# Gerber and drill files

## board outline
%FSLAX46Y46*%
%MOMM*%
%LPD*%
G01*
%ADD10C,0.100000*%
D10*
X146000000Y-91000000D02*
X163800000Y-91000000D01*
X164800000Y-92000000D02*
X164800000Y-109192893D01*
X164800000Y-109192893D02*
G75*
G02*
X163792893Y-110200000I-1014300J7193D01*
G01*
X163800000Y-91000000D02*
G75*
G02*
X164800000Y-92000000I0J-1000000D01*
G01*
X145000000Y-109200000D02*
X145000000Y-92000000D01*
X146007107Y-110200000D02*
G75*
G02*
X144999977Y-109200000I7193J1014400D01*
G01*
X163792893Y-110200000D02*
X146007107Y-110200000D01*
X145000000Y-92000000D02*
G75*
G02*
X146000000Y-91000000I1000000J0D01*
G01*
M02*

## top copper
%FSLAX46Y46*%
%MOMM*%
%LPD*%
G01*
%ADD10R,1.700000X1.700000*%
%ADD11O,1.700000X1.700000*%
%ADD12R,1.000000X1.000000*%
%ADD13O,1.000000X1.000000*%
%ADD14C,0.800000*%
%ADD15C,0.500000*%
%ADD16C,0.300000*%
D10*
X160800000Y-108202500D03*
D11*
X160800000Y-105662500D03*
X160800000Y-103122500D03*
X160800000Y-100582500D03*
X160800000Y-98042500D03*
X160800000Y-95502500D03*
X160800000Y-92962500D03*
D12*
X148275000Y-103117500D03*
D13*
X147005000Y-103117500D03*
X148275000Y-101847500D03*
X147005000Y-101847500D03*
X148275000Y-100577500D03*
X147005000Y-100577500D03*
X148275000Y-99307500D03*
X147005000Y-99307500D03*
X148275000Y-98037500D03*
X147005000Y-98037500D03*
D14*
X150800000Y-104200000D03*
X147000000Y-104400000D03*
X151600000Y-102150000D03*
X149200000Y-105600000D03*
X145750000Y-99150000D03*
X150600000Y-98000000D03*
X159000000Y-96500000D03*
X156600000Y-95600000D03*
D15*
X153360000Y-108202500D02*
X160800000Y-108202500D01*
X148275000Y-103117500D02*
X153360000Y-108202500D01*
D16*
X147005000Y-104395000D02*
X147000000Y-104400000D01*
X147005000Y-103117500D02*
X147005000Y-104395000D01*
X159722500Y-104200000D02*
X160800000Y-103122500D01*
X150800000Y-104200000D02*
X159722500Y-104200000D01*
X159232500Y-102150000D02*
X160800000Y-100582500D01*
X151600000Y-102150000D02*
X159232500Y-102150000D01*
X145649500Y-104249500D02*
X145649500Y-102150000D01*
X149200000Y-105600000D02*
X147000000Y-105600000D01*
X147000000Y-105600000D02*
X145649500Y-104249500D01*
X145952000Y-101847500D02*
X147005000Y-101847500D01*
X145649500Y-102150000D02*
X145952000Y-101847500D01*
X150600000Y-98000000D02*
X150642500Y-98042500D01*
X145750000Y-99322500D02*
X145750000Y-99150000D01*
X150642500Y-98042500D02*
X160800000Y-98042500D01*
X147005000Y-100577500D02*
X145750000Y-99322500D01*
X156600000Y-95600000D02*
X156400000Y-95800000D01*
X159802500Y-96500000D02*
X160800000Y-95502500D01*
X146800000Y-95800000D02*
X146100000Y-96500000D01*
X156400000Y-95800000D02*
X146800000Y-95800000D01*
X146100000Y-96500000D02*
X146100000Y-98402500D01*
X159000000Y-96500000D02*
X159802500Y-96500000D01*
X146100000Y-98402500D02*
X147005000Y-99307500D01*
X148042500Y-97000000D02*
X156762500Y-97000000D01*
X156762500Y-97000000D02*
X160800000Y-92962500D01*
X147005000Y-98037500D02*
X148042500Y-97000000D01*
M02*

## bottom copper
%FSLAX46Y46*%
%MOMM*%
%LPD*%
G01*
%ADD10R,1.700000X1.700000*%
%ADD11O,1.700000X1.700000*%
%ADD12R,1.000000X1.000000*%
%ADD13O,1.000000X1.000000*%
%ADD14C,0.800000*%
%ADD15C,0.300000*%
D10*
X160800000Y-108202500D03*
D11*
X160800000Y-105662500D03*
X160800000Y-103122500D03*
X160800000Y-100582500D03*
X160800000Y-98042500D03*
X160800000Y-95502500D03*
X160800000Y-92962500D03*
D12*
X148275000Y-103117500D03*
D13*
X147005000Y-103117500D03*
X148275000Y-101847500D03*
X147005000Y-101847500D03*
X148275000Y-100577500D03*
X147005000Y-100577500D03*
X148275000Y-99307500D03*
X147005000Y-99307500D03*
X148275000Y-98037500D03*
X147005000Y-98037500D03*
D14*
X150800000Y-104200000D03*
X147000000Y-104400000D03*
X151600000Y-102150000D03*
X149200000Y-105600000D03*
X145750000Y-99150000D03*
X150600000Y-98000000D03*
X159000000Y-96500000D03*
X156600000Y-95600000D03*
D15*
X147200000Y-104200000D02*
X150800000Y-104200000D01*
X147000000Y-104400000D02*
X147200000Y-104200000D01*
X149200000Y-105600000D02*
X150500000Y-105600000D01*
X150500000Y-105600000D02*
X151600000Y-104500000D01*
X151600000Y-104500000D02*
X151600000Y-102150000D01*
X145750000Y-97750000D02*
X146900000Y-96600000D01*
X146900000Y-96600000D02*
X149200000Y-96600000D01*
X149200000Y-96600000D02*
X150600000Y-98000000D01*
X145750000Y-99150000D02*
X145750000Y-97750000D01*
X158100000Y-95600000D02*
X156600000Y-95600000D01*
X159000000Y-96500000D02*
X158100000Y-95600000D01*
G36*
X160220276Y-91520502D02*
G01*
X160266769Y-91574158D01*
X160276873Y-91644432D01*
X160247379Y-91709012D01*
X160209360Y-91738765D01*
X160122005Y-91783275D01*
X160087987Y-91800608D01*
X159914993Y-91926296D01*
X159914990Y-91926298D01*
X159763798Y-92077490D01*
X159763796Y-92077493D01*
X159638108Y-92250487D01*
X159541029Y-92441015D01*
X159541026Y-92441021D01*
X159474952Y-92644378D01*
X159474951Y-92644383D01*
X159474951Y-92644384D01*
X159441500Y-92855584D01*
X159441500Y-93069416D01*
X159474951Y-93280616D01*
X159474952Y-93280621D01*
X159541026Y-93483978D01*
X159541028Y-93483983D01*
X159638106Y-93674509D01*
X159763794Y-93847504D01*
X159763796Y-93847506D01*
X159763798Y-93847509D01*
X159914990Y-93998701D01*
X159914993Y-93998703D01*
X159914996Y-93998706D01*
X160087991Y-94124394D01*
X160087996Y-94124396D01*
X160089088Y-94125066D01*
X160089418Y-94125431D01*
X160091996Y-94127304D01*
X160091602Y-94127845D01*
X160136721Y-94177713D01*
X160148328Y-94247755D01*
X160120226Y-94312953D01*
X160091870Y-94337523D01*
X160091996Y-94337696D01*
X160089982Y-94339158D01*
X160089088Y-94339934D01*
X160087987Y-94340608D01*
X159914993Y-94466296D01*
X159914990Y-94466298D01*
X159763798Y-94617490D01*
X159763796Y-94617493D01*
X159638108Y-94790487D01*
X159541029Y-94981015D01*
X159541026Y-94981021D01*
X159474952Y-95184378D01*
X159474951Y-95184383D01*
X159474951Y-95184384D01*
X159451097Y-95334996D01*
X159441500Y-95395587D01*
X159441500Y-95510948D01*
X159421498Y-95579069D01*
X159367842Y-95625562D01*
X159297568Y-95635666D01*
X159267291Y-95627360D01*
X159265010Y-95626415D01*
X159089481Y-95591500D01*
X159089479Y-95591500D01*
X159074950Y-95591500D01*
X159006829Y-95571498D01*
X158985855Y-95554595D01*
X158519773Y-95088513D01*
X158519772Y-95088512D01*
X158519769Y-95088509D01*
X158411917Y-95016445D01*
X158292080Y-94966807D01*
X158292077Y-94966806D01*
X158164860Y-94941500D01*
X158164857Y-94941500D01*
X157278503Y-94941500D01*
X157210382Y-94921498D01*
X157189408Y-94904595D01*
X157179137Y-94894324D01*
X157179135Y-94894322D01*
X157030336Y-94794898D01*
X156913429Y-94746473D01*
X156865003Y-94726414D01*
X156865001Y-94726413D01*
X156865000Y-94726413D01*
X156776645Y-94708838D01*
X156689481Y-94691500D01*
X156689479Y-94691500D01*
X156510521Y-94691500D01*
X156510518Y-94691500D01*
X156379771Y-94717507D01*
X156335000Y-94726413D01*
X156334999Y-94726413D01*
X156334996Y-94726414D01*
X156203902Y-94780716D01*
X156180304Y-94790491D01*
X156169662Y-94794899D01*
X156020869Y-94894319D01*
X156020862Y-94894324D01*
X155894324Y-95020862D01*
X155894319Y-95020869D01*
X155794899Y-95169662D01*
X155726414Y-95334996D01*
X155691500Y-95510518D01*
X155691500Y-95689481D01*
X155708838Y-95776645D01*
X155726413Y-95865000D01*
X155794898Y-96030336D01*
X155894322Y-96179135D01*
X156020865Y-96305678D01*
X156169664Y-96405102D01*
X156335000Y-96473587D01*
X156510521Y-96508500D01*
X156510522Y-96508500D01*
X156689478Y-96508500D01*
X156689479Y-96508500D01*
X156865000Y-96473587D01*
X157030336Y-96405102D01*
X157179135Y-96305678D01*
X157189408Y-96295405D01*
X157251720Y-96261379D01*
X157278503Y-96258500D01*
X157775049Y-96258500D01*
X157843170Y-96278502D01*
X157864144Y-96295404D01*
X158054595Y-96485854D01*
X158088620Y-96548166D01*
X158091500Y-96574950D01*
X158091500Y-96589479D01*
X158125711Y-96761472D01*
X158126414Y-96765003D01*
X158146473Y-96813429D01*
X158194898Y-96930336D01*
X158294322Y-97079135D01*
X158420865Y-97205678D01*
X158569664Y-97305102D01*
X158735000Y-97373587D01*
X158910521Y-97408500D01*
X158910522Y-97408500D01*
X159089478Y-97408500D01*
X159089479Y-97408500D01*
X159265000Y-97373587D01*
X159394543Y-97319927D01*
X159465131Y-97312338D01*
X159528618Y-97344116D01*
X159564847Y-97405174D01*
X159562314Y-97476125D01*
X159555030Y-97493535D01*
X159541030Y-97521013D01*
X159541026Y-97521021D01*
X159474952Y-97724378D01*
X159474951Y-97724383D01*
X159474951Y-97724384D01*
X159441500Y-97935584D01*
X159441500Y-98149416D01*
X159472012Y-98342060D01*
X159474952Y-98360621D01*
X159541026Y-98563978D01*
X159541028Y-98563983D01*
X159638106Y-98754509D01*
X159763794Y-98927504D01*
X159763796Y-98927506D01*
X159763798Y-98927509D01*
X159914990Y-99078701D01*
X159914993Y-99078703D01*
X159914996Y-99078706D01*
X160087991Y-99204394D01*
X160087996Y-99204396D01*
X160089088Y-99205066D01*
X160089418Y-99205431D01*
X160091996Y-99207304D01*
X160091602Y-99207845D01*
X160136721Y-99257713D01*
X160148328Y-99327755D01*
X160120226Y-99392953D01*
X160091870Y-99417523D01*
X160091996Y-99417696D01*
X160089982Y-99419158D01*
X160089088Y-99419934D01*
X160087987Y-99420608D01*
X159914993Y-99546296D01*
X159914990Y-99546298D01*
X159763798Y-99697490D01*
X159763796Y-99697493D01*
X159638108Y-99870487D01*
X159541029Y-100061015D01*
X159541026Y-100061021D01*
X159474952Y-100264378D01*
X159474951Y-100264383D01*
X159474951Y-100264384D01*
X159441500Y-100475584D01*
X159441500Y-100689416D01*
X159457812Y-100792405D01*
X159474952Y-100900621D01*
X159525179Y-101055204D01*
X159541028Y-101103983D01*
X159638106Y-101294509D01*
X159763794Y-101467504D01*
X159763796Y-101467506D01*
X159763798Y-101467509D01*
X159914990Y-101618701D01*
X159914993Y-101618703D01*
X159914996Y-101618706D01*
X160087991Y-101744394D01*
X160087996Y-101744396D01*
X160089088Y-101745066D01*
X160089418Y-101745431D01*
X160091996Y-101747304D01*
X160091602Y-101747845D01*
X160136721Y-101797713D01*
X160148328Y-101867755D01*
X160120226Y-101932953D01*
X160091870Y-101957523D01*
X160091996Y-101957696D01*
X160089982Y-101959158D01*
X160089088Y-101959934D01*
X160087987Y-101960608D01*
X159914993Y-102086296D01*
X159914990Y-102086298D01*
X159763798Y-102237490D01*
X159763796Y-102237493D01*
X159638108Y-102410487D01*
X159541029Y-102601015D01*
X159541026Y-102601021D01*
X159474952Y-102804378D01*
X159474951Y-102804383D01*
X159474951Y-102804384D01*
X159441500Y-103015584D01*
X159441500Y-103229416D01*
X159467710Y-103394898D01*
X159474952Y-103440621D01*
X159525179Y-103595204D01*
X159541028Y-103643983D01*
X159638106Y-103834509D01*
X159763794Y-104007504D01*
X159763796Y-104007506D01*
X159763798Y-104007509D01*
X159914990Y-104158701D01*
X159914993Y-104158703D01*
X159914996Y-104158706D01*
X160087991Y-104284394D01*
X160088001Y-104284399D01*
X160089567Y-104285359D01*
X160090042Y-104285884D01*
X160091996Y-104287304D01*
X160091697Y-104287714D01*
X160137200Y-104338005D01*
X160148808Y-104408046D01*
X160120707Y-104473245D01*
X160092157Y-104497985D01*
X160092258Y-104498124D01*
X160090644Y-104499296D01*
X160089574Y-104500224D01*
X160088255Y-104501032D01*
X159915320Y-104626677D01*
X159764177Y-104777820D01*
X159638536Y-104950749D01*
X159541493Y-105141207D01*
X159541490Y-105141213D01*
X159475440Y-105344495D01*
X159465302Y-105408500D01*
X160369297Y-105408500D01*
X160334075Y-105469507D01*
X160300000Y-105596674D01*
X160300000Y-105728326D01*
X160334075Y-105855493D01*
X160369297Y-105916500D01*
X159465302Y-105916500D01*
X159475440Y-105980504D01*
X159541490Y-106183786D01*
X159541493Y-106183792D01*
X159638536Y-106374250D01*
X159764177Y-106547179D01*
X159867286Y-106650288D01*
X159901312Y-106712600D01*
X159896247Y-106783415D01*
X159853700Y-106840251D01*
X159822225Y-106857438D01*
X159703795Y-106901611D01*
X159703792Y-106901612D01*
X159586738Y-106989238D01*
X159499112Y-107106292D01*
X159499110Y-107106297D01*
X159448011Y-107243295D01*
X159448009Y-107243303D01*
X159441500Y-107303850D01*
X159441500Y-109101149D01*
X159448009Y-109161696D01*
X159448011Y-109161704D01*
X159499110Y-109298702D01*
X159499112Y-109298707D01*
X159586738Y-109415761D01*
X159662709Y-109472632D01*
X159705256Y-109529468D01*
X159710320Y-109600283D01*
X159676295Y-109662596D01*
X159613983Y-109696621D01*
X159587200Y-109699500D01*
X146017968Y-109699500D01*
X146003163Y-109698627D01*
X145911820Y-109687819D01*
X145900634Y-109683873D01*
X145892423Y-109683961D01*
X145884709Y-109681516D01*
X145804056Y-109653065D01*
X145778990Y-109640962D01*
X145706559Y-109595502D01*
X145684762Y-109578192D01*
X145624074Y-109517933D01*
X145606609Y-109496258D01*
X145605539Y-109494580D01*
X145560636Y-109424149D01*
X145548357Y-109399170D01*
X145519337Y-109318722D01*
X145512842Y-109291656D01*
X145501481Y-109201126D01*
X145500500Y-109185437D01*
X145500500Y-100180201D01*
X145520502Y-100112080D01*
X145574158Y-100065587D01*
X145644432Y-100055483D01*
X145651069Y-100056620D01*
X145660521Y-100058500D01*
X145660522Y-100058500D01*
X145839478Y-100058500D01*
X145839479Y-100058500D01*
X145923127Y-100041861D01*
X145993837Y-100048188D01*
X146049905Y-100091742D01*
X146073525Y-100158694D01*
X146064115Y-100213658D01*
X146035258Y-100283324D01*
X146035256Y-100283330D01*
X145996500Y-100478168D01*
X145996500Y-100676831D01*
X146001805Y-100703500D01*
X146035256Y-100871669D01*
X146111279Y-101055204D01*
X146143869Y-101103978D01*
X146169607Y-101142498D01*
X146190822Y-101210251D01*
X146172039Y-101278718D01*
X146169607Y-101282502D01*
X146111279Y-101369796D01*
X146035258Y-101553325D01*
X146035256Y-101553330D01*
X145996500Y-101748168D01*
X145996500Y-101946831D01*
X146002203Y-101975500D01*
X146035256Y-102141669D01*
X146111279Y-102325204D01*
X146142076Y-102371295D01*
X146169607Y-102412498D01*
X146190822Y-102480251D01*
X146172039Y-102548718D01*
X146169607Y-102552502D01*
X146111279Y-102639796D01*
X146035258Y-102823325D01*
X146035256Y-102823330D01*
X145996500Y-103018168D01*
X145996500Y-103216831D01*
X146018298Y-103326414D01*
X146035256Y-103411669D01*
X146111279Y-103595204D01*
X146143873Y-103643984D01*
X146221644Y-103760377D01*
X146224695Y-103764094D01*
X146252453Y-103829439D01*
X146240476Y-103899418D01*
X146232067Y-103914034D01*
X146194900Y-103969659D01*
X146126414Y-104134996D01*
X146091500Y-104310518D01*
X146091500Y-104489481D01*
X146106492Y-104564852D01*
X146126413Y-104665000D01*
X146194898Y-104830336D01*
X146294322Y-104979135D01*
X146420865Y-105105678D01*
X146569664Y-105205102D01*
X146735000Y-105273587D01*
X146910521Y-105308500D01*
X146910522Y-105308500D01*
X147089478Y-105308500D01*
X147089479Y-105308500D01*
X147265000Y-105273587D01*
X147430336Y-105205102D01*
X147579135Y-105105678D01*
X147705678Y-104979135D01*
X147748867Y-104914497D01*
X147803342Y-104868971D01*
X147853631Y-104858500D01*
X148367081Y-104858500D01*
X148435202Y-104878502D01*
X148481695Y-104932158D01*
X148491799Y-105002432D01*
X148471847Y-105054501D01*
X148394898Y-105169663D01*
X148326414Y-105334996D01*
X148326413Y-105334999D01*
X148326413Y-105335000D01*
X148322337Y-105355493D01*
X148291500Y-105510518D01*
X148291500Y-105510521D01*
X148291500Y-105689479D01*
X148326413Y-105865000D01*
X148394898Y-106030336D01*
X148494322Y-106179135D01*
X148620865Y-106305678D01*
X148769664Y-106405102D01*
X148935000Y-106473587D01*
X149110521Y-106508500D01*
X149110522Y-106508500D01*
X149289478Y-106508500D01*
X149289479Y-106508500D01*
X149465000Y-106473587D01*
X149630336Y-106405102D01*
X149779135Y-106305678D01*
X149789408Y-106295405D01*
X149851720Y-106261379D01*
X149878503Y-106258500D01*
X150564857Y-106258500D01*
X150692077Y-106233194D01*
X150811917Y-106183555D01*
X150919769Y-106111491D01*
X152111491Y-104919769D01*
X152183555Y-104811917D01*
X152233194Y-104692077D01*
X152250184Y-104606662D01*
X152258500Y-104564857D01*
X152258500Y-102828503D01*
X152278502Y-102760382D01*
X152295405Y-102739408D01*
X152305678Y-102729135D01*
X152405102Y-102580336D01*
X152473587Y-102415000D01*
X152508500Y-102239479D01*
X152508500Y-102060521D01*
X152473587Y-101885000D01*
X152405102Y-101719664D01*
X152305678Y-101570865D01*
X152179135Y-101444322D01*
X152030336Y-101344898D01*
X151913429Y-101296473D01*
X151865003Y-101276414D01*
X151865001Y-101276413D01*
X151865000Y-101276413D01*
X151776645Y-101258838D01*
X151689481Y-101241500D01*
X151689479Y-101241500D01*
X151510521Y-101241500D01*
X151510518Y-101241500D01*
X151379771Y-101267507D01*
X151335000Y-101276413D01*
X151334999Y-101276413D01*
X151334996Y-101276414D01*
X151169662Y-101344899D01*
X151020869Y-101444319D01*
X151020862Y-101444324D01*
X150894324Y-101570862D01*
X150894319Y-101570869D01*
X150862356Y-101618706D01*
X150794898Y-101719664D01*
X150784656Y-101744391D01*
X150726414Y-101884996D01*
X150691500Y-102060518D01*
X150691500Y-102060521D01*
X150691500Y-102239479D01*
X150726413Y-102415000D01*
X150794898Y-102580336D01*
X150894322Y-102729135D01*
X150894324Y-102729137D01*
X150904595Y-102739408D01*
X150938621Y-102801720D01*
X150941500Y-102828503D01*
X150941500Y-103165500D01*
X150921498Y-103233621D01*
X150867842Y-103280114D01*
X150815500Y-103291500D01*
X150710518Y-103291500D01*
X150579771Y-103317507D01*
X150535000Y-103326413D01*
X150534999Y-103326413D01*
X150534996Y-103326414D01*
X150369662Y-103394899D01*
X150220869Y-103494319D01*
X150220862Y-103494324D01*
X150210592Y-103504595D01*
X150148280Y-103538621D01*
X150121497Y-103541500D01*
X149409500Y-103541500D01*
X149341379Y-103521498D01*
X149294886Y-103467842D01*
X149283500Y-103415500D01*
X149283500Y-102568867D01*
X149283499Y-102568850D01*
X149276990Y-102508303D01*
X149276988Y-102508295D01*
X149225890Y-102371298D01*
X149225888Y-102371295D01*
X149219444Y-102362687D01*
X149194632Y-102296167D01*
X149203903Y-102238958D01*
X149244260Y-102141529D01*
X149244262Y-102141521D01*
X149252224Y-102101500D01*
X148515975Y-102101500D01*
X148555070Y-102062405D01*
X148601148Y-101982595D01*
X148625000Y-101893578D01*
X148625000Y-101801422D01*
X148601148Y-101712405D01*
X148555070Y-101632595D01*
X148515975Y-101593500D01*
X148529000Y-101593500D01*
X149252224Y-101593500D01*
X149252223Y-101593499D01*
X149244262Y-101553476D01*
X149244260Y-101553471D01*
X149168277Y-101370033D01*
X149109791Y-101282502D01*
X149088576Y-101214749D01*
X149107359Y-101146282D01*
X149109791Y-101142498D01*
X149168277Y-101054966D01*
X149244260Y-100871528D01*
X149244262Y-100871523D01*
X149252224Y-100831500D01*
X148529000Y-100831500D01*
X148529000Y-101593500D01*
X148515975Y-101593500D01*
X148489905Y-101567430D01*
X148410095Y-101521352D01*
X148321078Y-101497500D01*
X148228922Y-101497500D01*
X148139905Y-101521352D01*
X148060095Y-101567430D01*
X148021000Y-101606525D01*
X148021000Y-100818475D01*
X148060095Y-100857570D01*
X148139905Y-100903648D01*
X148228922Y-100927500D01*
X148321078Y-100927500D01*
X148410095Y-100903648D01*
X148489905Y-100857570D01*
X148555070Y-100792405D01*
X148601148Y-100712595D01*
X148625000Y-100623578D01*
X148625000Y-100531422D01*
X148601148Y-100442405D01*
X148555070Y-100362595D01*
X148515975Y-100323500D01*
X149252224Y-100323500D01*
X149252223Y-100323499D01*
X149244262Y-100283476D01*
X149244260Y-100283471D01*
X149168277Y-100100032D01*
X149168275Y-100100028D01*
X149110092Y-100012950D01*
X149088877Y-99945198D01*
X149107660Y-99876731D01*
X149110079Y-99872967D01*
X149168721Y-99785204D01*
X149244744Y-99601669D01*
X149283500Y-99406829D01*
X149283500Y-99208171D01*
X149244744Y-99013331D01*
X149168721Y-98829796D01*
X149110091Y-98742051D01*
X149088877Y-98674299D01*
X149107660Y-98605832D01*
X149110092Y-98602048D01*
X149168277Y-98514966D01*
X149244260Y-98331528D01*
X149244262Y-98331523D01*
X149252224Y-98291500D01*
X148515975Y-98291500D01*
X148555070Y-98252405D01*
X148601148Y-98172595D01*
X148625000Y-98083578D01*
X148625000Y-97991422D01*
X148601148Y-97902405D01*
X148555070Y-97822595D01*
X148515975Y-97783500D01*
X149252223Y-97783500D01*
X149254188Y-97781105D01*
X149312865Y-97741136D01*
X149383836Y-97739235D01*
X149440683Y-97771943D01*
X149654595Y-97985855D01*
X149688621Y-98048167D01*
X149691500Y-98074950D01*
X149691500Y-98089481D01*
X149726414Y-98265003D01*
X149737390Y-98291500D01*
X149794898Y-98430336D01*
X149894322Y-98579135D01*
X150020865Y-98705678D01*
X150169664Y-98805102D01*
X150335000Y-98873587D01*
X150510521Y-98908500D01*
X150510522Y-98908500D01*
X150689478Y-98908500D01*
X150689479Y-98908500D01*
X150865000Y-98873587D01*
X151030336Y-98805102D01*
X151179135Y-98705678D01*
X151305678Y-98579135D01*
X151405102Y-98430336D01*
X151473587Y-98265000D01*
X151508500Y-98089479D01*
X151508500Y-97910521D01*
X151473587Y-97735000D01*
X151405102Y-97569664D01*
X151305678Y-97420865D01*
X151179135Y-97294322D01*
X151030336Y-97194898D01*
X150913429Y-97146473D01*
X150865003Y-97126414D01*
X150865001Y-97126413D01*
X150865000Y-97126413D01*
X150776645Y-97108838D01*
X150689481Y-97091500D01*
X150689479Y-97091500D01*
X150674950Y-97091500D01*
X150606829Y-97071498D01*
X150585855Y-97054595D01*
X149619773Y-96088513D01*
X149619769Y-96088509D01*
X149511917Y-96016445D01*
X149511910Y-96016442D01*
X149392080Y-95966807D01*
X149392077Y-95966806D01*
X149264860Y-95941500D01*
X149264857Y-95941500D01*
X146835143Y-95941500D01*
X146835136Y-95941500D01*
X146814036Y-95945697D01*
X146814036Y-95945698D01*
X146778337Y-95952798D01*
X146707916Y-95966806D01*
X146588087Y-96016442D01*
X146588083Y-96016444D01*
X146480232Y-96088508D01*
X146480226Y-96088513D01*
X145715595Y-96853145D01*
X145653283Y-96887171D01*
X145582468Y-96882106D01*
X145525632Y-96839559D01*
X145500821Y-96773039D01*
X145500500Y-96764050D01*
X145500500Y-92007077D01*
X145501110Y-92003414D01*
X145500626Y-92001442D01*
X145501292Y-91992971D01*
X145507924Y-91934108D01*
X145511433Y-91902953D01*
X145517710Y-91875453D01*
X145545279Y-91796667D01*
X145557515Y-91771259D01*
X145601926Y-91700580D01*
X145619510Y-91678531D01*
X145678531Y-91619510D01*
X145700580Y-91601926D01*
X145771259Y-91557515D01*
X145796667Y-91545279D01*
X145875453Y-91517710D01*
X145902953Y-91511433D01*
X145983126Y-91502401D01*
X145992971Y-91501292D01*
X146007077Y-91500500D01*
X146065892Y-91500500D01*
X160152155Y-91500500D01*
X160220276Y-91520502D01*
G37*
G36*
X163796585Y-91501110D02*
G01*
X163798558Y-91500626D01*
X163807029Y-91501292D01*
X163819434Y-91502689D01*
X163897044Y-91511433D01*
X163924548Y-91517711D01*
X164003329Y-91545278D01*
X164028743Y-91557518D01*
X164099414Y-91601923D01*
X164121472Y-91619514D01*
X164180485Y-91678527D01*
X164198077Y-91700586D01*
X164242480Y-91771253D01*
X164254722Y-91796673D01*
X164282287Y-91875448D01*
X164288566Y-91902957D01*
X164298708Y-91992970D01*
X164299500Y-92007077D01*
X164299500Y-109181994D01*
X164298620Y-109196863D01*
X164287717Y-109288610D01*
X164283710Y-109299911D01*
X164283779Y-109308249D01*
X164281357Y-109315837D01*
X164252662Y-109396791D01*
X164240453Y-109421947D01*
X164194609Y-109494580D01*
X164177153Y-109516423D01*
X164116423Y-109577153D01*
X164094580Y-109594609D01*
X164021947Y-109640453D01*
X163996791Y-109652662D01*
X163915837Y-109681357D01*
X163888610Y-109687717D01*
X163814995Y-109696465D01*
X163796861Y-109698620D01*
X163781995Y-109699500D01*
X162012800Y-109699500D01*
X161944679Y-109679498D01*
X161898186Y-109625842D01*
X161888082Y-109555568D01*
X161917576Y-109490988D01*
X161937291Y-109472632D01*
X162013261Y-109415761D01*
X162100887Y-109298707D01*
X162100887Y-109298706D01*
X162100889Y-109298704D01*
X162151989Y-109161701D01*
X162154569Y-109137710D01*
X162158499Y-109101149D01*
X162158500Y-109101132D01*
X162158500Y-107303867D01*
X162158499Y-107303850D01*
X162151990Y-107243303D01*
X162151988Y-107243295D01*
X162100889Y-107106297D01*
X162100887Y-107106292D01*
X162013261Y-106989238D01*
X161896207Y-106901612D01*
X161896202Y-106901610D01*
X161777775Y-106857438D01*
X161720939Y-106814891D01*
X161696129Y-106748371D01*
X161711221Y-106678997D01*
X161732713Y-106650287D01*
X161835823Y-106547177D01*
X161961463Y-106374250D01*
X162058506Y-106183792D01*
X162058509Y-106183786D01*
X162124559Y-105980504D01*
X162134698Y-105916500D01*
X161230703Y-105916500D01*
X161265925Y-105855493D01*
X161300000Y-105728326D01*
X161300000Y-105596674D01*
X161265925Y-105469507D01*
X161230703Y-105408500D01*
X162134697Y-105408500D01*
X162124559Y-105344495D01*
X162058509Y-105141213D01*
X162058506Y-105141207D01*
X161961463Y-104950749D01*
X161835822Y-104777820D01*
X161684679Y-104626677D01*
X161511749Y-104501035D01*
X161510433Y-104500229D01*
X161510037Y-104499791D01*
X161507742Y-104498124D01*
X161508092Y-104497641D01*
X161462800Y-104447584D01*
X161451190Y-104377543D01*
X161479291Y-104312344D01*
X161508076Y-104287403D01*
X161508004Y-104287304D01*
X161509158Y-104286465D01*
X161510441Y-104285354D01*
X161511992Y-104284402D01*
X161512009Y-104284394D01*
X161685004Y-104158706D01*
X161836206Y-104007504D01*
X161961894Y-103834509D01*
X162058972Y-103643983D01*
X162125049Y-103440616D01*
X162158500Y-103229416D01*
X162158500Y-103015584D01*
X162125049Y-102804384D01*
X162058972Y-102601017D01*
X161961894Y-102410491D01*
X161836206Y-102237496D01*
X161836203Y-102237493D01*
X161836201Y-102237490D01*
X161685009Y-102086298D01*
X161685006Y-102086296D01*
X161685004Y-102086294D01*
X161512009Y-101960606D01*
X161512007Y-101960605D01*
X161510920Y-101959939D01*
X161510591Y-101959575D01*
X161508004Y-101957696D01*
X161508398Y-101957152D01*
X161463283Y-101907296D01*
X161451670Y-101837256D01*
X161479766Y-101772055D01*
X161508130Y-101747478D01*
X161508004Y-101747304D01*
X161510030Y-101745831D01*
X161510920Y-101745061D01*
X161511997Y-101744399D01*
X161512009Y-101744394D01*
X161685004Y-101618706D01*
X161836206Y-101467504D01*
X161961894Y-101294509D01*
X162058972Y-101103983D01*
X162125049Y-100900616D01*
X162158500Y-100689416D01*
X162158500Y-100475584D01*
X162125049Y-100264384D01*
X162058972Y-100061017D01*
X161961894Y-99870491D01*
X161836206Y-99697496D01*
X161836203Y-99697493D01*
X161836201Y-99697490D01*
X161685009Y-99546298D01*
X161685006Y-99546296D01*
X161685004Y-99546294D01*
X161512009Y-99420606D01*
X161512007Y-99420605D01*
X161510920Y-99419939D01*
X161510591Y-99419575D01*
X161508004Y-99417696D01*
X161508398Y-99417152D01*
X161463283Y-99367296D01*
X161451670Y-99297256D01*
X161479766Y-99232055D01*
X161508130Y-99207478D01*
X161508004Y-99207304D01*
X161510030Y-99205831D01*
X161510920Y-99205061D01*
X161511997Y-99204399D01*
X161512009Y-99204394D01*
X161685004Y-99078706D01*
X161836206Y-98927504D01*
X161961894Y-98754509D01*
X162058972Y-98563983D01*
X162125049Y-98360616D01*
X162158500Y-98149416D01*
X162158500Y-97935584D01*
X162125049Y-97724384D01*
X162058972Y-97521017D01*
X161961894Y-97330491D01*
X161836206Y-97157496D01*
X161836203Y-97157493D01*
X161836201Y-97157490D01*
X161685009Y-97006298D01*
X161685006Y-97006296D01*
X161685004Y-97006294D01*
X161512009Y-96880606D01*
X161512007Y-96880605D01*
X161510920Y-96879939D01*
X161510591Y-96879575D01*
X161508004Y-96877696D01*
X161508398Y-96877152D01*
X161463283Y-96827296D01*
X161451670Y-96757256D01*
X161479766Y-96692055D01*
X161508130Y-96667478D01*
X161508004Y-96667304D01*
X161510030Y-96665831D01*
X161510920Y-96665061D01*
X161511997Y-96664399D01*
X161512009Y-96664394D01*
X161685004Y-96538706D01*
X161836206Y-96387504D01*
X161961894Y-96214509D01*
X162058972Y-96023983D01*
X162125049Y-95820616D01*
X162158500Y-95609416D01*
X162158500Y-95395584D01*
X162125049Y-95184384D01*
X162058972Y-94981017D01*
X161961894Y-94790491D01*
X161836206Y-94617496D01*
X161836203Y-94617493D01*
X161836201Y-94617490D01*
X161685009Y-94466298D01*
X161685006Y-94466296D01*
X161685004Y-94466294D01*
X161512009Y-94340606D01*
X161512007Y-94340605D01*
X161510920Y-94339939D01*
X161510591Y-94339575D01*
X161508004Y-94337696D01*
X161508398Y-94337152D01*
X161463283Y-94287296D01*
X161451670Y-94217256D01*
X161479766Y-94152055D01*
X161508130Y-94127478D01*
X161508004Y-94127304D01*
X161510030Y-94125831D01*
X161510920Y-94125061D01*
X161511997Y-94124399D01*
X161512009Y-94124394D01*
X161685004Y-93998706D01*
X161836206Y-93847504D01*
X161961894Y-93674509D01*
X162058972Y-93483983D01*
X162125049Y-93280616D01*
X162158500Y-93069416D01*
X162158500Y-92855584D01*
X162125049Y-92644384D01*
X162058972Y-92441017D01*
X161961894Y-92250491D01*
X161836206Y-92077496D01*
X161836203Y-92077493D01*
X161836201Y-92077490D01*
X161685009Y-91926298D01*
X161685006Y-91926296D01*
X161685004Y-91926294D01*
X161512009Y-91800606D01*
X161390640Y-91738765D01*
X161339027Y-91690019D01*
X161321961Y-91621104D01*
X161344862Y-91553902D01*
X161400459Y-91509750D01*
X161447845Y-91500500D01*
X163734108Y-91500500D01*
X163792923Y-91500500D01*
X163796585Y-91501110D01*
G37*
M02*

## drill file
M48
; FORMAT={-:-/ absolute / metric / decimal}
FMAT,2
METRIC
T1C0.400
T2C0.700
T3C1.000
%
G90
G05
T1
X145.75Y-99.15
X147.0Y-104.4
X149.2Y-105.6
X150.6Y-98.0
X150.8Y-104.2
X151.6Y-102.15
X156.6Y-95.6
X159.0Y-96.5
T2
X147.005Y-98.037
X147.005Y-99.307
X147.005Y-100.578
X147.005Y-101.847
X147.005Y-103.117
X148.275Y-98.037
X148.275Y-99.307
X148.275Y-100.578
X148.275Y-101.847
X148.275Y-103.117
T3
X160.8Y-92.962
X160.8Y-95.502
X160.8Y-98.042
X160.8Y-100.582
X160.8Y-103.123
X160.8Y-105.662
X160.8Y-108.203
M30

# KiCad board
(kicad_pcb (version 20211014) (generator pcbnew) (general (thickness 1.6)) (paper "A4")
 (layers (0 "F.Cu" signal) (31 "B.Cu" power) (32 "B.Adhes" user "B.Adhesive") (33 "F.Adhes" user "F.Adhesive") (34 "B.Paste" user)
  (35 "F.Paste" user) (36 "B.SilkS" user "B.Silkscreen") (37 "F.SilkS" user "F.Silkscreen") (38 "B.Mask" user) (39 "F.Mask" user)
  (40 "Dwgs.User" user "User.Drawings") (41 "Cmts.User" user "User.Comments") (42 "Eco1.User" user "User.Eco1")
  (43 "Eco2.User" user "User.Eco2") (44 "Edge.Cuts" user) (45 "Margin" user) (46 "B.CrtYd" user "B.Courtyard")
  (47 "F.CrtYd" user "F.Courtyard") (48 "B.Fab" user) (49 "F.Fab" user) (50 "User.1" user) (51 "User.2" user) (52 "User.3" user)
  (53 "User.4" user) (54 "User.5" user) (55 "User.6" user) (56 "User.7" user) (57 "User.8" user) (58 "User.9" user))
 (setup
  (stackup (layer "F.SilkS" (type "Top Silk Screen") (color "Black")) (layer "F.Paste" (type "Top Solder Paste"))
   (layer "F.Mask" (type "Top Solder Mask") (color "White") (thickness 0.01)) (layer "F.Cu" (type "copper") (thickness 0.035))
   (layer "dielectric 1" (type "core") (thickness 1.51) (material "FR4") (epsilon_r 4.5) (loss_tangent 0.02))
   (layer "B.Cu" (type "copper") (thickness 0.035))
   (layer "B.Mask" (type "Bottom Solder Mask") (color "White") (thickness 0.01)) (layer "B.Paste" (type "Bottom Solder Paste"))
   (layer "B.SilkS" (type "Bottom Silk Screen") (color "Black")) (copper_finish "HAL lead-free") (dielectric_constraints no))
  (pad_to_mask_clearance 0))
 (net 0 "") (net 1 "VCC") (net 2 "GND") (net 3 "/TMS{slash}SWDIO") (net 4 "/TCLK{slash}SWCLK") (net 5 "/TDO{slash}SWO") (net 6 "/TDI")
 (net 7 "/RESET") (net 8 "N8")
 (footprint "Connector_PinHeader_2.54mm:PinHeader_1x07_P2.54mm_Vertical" (layer "F.Cu") (at 160.8 108.2025 180)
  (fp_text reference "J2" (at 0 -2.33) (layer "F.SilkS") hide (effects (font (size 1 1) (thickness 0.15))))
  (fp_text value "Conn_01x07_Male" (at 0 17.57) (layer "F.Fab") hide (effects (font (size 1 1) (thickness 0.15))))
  (pad "1" thru_hole rect (at 0 0 180) (size 1.7 1.7) (drill 1) (layers *.Cu *.Mask) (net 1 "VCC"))
  (pad "2" thru_hole oval (at 0 2.54 180) (size 1.7 1.7) (drill 1) (layers *.Cu *.Mask) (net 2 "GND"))
  (pad "3" thru_hole oval (at 0 5.08 180) (size 1.7 1.7) (drill 1) (layers *.Cu *.Mask) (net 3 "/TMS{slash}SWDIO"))
  (pad "4" thru_hole oval (at 0 7.62 180) (size 1.7 1.7) (drill 1) (layers *.Cu *.Mask) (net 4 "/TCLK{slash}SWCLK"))
  (pad "5" thru_hole oval (at 0 10.16 180) (size 1.7 1.7) (drill 1) (layers *.Cu *.Mask) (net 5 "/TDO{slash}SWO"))
  (pad "6" thru_hole oval (at 0 12.7 180) (size 1.7 1.7) (drill 1) (layers *.Cu *.Mask) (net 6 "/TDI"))
  (pad "7" thru_hole oval (at 0 15.24 180) (size 1.7 1.7) (drill 1) (layers *.Cu *.Mask) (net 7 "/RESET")))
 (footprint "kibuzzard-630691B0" (layer "F.Cu") (at 157.3 108.2)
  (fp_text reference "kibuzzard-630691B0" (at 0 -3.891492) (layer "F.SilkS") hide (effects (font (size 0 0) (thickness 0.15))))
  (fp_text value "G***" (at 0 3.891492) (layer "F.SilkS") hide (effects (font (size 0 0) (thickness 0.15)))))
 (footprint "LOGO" (layer "B.Cu") (at 148.199134 94.2 90)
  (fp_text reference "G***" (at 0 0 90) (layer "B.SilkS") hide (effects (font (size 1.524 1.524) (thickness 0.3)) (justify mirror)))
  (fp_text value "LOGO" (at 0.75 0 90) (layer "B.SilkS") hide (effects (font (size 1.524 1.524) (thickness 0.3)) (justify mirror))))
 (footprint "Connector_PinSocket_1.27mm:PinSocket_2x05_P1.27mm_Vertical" (layer "B.Cu") (at 148.275 103.1175)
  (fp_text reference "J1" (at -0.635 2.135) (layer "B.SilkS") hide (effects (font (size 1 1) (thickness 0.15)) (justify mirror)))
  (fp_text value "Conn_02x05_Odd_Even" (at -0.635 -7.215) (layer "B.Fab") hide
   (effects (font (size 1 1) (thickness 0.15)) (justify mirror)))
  (pad "1" thru_hole rect (at 0 0) (size 1 1) (drill 0.7) (layers *.Cu *.Mask) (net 1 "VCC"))
  (pad "2" thru_hole oval (at -1.27 0) (size 1 1) (drill 0.7) (layers *.Cu *.Mask) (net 3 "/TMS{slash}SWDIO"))
  (pad "3" thru_hole oval (at 0 -1.27) (size 1 1) (drill 0.7) (layers *.Cu *.Mask) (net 2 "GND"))
  (pad "4" thru_hole oval (at -1.27 -1.27) (size 1 1) (drill 0.7) (layers *.Cu *.Mask) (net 4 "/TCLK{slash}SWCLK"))
  (pad "5" thru_hole oval (at 0 -2.54) (size 1 1) (drill 0.7) (layers *.Cu *.Mask) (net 2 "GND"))
  (pad "6" thru_hole oval (at -1.27 -2.54) (size 1 1) (drill 0.7) (layers *.Cu *.Mask) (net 5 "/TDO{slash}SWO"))
  (pad "7" thru_hole oval (at 0 -3.81) (size 1 1) (drill 0.7) (layers *.Cu *.Mask) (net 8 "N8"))
  (pad "8" thru_hole oval (at -1.27 -3.81) (size 1 1) (drill 0.7) (layers *.Cu *.Mask) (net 6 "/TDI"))
  (pad "9" thru_hole oval (at 0 -5.08) (size 1 1) (drill 0.7) (layers *.Cu *.Mask) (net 2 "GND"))
  (pad "10" thru_hole oval (at -1.27 -5.08) (size 1 1) (drill 0.7) (layers *.Cu *.Mask) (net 7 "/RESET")))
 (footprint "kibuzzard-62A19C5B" (layer "B.Cu") (at 154.1 100.5775 90)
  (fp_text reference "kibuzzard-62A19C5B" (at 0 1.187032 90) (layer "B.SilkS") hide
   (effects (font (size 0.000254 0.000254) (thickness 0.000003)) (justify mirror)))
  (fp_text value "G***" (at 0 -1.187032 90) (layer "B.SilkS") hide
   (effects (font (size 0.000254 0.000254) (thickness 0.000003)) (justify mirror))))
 (gr_line (start 146 91) (end 163.8 91) (layer "Edge.Cuts") (width 0.1))
 (gr_line (start 164.8 92) (end 164.8 109.192893) (layer "Edge.Cuts") (width 0.1))
 (gr_arc (start 164.8 109.192893) (mid 164.502939 109.902939) (end 163.792893 110.2) (layer "Edge.Cuts") (width 0.1))
 (gr_arc (start 163.8 91) (mid 164.507107 91.292893) (end 164.8 92) (layer "Edge.Cuts") (width 0.1))
 (gr_line (start 145 109.2) (end 145 92) (layer "Edge.Cuts") (width 0.1))
 (gr_arc (start 146.007107 110.2) (mid 145.299551 109.905452) (end 145 109.2) (layer "Edge.Cuts") (width 0.1))
 (gr_line (start 163.792893 110.2) (end 146.007107 110.2) (layer "Edge.Cuts") (width 0.1))
 (gr_arc (start 145 92) (mid 145.292893 91.292893) (end 146 91) (layer "Edge.Cuts") (width 0.1))
 (segment (start 153.36 108.2025) (end 160.8 108.2025) (width 0.5) (layer "F.Cu") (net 1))
 (segment (start 148.275 103.1175) (end 153.36 108.2025) (width 0.5) (layer "F.Cu") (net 1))
 (segment (start 147.005 104.395) (end 147 104.4) (width 0.3) (layer "F.Cu") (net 3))
 (segment (start 147.005 103.1175) (end 147.005 104.395) (width 0.3) (layer "F.Cu") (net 3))
 (segment (start 159.7225 104.2) (end 160.8 103.1225) (width 0.3) (layer "F.Cu") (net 3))
 (segment (start 150.8 104.2) (end 159.7225 104.2) (width 0.3) (layer "F.Cu") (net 3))
 (via (at 150.8 104.2) (size 0.8) (drill 0.4) (layers "F.Cu" "B.Cu") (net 3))
 (via (at 147 104.4) (size 0.8) (drill 0.4) (layers "F.Cu" "B.Cu") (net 3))
 (segment (start 147.2 104.2) (end 150.8 104.2) (width 0.3) (layer "B.Cu") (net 3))
 (segment (start 147 104.4) (end 147.2 104.2) (width 0.3) (layer "B.Cu") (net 3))
 (segment (start 159.2325 102.15) (end 160.8 100.5825) (width 0.3) (layer "F.Cu") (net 4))
 (segment (start 151.6 102.15) (end 159.2325 102.15) (width 0.3) (layer "F.Cu") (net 4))
 (segment (start 145.6495 104.2495) (end 145.6495 102.15) (width 0.3) (layer "F.Cu") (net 4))
 (segment (start 149.2 105.6) (end 147 105.6) (width 0.3) (layer "F.Cu") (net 4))
 (segment (start 147 105.6) (end 145.6495 104.2495) (width 0.3) (layer "F.Cu") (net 4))
 (segment (start 145.952 101.8475) (end 147.005 101.8475) (width 0.3) (layer "F.Cu") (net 4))
 (segment (start 145.6495 102.15) (end 145.952 101.8475) (width 0.3) (layer "F.Cu") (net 4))
 (via (at 151.6 102.15) (size 0.8) (drill 0.4) (layers "F.Cu" "B.Cu") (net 4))
 (via (at 149.2 105.6) (size 0.8) (drill 0.4) (layers "F.Cu" "B.Cu") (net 4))
 (segment (start 149.2 105.6) (end 150.5 105.6) (width 0.3) (layer "B.Cu") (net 4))
 (segment (start 150.5 105.6) (end 151.6 104.5) (width 0.3) (layer "B.Cu") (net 4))
 (segment (start 151.6 104.5) (end 151.6 102.15) (width 0.3) (layer "B.Cu") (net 4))
 (segment (start 150.6 98) (end 150.6425 98.0425) (width 0.3) (layer "F.Cu") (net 5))
 (segment (start 145.75 99.3225) (end 145.75 99.15) (width 0.3) (layer "F.Cu") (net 5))
 (segment (start 150.6425 98.0425) (end 160.8 98.0425) (width 0.3) (layer "F.Cu") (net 5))
 (segment (start 147.005 100.5775) (end 145.75 99.3225) (width 0.3) (layer "F.Cu") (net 5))
 (via (at 145.75 99.15) (size 0.8) (drill 0.4) (layers "F.Cu" "B.Cu") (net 5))
 (via (at 150.6 98) (size 0.8) (drill 0.4) (layers "F.Cu" "B.Cu") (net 5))
 (segment (start 145.75 97.75) (end 146.9 96.6) (width 0.3) (layer "B.Cu") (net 5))
 (segment (start 146.9 96.6) (end 149.2 96.6) (width 0.3) (layer "B.Cu") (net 5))
 (segment (start 149.2 96.6) (end 150.6 98) (width 0.3) (layer "B.Cu") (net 5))
 (segment (start 145.75 99.15) (end 145.75 97.75) (width 0.3) (layer "B.Cu") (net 5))
 (segment (start 156.6 95.6) (end 156.4 95.8) (width 0.3) (layer "F.Cu") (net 6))
 (segment (start 159.8025 96.5) (end 160.8 95.5025) (width 0.3) (layer "F.Cu") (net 6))
 (segment (start 146.8 95.8) (end 146.1 96.5) (width 0.3) (layer "F.Cu") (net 6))
 (segment (start 156.4 95.8) (end 146.8 95.8) (width 0.3) (layer "F.Cu") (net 6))
 (segment (start 146.1 96.5) (end 146.1 98.4025) (width 0.3) (layer "F.Cu") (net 6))
 (segment (start 159 96.5) (end 159.8025 96.5) (width 0.3) (layer "F.Cu") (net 6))
 (segment (start 146.1 98.4025) (end 147.005 99.3075) (width 0.3) (layer "F.Cu") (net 6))
 (via (at 159 96.5) (size 0.8) (drill 0.4) (layers "F.Cu" "B.Cu") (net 6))
 (via (at 156.6 95.6) (size 0.8) (drill 0.4) (layers "F.Cu" "B.Cu") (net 6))
 (segment (start 158.1 95.6) (end 156.6 95.6) (width 0.3) (layer "B.Cu") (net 6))
 (segment (start 159 96.5) (end 158.1 95.6) (width 0.3) (layer "B.Cu") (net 6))
 (segment (start 148.0425 97) (end 156.7625 97) (width 0.3) (layer "F.Cu") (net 7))
 (segment (start 156.7625 97) (end 160.8 92.9625) (width 0.3) (layer "F.Cu") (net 7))
 (segment (start 147.005 98.0375) (end 148.0425 97) (width 0.3) (layer "F.Cu") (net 7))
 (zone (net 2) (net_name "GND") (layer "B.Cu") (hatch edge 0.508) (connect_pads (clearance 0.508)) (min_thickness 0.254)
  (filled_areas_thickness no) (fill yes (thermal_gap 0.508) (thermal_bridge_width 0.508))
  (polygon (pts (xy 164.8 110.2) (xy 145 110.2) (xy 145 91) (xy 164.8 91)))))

